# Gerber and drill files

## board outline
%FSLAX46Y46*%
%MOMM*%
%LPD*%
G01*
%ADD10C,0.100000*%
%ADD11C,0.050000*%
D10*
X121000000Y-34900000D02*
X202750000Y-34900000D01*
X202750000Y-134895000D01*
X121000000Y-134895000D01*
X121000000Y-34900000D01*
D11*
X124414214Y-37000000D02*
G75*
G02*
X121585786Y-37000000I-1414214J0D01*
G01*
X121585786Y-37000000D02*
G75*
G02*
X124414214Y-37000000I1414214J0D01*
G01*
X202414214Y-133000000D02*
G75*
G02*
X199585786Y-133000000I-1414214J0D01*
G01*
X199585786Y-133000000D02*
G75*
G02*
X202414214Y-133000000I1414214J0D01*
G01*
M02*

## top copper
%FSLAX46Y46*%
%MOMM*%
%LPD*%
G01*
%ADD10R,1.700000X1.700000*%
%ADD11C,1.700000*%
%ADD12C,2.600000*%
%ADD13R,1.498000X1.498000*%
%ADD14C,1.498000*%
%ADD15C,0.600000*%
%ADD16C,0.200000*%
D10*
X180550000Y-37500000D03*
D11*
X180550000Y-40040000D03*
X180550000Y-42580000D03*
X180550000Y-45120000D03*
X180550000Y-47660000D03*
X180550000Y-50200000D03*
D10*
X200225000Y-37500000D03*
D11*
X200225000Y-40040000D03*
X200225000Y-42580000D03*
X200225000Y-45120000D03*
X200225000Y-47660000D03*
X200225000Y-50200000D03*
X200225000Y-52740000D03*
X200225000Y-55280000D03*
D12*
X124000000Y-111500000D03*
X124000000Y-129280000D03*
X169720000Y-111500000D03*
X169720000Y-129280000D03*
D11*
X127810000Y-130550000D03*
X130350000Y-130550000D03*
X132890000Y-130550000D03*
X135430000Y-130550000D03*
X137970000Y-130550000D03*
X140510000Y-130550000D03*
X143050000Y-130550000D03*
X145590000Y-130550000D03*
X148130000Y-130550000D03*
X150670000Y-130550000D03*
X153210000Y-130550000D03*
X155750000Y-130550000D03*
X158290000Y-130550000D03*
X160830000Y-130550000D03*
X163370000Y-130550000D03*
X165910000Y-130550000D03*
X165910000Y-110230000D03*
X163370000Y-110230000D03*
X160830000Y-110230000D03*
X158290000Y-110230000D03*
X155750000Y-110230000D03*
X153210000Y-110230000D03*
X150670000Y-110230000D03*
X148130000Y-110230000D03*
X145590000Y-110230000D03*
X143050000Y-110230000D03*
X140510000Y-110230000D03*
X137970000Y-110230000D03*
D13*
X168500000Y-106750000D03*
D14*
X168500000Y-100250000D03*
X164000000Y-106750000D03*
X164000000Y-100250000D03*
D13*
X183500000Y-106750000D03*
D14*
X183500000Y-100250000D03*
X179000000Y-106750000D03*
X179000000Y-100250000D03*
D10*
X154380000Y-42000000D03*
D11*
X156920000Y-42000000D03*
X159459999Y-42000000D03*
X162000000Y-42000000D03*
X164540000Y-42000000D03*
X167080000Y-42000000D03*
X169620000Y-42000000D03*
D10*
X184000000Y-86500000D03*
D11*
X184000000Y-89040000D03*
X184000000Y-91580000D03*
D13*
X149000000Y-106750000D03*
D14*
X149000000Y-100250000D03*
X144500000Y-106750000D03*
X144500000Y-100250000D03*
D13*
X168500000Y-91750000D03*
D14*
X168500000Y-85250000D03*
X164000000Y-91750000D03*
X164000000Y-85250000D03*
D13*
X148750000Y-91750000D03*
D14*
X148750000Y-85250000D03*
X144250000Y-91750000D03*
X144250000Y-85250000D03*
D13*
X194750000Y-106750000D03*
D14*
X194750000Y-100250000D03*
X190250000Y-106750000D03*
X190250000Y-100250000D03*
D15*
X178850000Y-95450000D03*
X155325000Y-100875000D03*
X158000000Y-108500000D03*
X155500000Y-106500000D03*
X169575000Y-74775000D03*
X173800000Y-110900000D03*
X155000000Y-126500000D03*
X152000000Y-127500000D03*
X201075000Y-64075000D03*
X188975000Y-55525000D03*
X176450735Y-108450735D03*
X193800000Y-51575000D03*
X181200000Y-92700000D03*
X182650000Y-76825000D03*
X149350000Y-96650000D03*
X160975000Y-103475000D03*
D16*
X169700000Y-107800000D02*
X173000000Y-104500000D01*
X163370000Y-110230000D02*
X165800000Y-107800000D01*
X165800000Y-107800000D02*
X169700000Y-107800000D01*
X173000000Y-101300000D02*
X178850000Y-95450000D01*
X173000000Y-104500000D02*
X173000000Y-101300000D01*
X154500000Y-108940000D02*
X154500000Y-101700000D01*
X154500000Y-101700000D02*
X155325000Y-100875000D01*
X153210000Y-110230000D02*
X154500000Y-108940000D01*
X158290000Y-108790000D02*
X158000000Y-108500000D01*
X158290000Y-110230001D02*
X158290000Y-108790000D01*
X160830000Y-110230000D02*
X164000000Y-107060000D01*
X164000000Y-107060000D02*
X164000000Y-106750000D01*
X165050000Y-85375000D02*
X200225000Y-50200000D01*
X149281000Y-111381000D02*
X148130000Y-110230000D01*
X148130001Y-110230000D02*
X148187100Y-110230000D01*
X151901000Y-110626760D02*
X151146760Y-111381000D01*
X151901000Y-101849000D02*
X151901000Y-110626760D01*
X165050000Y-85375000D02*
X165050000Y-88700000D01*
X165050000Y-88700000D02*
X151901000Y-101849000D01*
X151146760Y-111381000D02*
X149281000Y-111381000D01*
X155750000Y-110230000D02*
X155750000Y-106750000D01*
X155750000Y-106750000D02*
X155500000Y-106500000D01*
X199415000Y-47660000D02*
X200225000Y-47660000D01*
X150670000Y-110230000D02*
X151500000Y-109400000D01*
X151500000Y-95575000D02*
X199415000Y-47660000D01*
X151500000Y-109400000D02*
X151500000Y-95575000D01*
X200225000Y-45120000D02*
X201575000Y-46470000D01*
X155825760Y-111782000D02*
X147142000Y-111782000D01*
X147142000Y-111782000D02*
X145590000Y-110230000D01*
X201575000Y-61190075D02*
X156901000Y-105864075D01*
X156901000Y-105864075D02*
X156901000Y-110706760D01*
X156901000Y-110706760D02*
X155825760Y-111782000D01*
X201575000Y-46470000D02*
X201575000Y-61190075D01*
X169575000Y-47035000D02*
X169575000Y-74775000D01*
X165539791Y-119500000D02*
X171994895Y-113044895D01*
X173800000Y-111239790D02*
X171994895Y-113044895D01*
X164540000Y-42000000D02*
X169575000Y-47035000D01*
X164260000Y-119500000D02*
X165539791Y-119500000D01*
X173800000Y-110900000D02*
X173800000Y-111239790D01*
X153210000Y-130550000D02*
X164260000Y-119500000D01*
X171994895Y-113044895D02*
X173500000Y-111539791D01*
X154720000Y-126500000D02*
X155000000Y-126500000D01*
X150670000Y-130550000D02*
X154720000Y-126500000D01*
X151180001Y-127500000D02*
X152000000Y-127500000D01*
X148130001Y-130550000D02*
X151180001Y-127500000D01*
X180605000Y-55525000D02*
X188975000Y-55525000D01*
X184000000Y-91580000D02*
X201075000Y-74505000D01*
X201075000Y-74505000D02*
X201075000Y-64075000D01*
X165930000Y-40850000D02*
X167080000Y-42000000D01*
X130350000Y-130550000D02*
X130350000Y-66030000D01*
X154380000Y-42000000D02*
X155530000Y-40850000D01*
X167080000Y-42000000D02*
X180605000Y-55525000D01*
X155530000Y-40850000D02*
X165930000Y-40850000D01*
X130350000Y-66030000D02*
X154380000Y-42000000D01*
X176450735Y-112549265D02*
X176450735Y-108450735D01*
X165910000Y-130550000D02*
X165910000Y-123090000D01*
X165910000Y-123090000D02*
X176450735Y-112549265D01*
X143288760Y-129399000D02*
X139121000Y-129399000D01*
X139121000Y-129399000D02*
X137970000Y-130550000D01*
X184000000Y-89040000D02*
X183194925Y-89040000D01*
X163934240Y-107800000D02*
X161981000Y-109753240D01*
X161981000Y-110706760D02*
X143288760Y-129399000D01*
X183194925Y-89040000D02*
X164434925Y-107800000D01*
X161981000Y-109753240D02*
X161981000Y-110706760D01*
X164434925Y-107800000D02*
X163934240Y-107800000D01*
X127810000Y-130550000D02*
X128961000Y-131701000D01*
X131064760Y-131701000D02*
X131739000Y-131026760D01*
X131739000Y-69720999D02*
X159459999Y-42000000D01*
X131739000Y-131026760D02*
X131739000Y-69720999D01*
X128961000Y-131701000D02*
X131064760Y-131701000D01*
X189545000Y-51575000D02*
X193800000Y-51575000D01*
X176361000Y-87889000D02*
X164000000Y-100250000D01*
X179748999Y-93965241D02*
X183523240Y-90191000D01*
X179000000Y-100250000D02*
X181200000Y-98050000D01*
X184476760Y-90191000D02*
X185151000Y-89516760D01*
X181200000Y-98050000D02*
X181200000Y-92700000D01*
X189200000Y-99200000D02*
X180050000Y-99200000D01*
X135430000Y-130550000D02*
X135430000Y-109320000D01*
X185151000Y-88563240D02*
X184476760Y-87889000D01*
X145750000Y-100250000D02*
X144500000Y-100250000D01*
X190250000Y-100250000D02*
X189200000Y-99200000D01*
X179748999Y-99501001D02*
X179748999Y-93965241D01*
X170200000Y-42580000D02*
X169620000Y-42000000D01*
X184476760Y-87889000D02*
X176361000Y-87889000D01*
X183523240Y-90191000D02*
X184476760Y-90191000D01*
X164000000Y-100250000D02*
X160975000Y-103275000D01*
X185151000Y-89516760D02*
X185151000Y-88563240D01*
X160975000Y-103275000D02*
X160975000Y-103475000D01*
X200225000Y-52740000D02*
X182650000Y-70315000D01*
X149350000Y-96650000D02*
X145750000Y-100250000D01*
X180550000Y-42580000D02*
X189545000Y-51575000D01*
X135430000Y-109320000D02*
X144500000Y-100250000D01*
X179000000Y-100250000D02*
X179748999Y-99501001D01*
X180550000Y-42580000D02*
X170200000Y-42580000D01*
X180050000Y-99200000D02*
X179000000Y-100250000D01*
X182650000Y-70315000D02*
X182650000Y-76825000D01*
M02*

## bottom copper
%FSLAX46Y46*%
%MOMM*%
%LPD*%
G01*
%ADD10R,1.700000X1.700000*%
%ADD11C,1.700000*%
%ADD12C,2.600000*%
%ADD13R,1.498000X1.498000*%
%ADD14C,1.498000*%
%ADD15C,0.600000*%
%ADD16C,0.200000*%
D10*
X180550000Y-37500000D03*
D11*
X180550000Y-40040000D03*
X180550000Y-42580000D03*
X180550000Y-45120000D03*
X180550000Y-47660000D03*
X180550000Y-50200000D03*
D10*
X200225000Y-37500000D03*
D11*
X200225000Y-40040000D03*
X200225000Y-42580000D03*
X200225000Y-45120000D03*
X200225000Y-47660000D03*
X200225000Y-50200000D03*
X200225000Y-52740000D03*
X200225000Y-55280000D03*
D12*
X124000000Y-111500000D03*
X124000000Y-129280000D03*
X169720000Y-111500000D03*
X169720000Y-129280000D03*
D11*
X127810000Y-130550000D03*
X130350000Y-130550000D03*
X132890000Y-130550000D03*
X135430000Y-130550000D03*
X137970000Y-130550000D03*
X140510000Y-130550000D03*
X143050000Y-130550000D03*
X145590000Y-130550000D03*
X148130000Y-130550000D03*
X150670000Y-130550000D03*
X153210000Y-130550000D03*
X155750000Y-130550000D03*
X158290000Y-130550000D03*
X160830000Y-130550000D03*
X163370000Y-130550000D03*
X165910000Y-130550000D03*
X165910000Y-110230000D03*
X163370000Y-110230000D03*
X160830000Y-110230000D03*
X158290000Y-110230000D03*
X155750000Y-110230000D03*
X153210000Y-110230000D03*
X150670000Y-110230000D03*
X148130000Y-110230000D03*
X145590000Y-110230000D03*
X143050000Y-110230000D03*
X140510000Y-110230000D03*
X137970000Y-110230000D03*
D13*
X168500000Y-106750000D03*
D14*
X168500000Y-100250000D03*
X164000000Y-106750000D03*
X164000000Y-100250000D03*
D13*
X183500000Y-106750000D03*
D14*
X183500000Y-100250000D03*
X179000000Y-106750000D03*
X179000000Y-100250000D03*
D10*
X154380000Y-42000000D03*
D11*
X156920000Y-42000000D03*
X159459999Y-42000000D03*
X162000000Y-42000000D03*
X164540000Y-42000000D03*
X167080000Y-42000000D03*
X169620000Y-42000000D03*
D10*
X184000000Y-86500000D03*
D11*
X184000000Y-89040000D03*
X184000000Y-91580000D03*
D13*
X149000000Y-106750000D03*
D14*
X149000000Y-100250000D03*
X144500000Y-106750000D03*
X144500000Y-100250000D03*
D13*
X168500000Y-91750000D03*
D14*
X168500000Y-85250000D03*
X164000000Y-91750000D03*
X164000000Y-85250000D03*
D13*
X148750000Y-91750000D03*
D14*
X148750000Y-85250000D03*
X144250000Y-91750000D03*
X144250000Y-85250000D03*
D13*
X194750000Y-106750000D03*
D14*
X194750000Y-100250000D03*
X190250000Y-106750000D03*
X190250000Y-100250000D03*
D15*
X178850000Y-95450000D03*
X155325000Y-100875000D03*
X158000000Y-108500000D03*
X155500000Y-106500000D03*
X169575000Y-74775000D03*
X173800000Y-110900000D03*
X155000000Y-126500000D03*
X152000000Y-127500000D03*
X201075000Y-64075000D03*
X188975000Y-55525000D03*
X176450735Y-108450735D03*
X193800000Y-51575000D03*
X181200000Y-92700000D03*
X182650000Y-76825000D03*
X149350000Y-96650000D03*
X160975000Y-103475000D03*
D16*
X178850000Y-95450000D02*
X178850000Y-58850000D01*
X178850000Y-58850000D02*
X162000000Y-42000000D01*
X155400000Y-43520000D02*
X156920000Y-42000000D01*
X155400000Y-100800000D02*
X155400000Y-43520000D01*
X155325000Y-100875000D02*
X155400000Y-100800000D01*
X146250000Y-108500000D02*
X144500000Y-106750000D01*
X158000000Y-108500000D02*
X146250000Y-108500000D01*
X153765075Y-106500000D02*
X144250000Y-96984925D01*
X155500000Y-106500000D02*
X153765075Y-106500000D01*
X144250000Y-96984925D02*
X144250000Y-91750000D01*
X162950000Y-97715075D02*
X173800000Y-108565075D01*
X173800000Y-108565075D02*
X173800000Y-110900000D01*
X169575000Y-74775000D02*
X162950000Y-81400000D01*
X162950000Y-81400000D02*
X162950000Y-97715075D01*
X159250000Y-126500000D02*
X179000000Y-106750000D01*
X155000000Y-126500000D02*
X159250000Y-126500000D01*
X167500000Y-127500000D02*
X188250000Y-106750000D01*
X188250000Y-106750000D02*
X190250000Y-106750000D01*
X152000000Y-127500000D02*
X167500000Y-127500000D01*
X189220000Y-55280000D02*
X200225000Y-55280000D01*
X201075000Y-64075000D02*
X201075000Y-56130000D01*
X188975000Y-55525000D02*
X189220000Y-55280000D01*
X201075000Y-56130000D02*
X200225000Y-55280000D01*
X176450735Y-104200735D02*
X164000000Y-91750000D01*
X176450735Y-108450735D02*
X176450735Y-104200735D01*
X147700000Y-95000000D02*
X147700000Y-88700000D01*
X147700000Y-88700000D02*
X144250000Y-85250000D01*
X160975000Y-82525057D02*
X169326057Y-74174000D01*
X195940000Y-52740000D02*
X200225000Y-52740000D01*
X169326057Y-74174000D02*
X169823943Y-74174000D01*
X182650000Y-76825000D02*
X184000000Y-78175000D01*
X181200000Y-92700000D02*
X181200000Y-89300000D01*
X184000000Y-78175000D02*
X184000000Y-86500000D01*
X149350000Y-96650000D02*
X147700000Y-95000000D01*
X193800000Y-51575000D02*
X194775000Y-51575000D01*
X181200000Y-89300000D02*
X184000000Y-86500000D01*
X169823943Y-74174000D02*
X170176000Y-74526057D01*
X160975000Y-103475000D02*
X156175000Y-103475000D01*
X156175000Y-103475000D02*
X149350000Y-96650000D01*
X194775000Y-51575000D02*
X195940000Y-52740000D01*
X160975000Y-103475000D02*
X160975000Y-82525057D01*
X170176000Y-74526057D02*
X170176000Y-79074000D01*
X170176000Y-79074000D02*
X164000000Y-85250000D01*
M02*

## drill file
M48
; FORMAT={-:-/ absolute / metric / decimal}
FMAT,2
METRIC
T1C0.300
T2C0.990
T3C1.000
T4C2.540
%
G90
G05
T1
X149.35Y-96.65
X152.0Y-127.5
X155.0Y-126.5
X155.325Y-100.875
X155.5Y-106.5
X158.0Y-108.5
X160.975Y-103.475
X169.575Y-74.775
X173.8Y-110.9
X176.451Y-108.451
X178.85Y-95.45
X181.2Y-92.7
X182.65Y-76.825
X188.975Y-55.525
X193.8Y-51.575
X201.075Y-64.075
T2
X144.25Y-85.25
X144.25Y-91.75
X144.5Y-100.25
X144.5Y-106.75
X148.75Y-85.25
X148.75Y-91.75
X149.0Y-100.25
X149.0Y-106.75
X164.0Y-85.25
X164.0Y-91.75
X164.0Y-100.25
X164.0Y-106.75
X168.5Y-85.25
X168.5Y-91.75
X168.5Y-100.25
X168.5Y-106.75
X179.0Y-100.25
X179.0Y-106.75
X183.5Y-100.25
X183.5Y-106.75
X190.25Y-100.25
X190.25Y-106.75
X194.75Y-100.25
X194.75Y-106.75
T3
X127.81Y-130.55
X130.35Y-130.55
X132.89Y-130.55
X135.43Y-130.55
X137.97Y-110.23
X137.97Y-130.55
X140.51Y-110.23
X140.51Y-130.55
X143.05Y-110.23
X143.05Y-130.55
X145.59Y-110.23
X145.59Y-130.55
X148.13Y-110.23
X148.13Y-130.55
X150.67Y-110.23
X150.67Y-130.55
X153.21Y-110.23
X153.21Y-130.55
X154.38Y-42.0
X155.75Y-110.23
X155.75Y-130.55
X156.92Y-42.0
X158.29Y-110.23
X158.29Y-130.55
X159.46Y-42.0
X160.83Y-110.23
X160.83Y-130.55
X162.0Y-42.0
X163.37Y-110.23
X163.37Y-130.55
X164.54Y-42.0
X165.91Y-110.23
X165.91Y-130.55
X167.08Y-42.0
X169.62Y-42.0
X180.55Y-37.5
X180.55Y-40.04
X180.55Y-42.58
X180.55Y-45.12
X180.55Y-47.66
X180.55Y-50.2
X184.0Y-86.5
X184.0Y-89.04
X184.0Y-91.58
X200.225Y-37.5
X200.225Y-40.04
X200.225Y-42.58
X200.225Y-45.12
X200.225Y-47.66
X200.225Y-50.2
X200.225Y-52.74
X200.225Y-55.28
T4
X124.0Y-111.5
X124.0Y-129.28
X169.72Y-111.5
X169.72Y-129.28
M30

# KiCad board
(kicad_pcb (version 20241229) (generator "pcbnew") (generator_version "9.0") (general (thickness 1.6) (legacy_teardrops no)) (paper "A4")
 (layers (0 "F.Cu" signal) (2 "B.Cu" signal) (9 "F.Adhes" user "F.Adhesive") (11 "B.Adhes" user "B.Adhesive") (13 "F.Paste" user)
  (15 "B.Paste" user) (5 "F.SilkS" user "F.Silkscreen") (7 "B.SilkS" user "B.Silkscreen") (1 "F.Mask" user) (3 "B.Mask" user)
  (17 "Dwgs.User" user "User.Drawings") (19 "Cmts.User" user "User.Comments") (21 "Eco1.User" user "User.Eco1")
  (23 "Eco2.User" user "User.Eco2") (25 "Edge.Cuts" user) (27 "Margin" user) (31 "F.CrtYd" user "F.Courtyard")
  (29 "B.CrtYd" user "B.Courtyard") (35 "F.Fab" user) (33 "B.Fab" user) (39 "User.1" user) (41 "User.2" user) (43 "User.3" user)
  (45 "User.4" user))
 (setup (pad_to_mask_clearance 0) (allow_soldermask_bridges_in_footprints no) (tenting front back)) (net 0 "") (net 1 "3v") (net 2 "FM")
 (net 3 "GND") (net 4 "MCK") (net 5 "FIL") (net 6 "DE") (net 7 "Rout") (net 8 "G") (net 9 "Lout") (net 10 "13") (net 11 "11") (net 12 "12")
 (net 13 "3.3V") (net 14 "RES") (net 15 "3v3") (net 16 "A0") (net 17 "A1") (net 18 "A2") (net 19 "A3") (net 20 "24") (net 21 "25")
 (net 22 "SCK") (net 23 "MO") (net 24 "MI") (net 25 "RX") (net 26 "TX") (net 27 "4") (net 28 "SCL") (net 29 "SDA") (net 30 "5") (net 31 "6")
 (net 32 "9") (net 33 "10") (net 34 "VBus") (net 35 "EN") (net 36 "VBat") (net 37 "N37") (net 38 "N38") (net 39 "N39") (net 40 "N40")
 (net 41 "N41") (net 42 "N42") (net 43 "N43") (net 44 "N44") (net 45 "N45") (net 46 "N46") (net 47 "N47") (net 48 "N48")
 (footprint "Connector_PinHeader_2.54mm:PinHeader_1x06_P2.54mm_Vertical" (layer "F.Cu") (at 180.55 37.5)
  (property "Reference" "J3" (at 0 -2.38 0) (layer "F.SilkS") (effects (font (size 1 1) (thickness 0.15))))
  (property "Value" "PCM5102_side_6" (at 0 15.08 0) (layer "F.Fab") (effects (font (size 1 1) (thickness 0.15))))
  (pad "1" thru_hole rect (at 0 0) (size 1.7 1.7) (drill 1) (layers "*.Cu" "*.Mask") (remove_unused_layers no) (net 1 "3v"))
  (pad "2" thru_hole circle (at 0 2.54) (size 1.7 1.7) (drill 1) (layers "*.Cu" "*.Mask") (remove_unused_layers no) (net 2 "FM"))
  (pad "3" thru_hole circle (at 0 5.08) (size 1.7 1.7) (drill 1) (layers "*.Cu" "*.Mask") (remove_unused_layers no) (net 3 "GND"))
  (pad "4" thru_hole circle (at 0 7.62) (size 1.7 1.7) (drill 1) (layers "*.Cu" "*.Mask") (remove_unused_layers no) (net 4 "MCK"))
  (pad "5" thru_hole circle (at 0 10.16) (size 1.7 1.7) (drill 1) (layers "*.Cu" "*.Mask") (remove_unused_layers no) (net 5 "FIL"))
  (pad "6" thru_hole circle (at 0 12.7) (size 1.7 1.7) (drill 1) (layers "*.Cu" "*.Mask") (remove_unused_layers no) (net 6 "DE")))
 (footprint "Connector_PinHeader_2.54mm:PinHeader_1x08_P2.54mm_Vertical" (layer "F.Cu") (at 200.225 37.5)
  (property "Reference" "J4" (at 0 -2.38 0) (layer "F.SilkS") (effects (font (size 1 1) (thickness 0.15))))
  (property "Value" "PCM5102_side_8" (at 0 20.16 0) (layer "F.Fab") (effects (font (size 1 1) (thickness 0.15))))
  (pad "1" thru_hole rect (at 0 0) (size 1.7 1.7) (drill 1) (layers "*.Cu" "*.Mask") (remove_unused_layers no) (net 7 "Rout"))
  (pad "2" thru_hole circle (at 0 2.54) (size 1.7 1.7) (drill 1) (layers "*.Cu" "*.Mask") (remove_unused_layers no) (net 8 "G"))
  (pad "3" thru_hole circle (at 0 5.08) (size 1.7 1.7) (drill 1) (layers "*.Cu" "*.Mask") (remove_unused_layers no) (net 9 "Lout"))
  (pad "4" thru_hole circle (at 0 7.62) (size 1.7 1.7) (drill 1) (layers "*.Cu" "*.Mask") (remove_unused_layers no) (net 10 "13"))
  (pad "5" thru_hole circle (at 0 10.16) (size 1.7 1.7) (drill 1) (layers "*.Cu" "*.Mask") (remove_unused_layers no) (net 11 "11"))
  (pad "6" thru_hole circle (at 0 12.7) (size 1.7 1.7) (drill 1) (layers "*.Cu" "*.Mask") (remove_unused_layers no) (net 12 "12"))
  (pad "7" thru_hole circle (at 0 15.24) (size 1.7 1.7) (drill 1) (layers "*.Cu" "*.Mask") (remove_unused_layers no) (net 3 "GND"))
  (pad "8" thru_hole circle (at 0 17.78) (size 1.7 1.7) (drill 1) (layers "*.Cu" "*.Mask") (remove_unused_layers no) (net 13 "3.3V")))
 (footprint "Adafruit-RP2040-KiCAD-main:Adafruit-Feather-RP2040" (layer "F.Cu") (at 146.86 120.39)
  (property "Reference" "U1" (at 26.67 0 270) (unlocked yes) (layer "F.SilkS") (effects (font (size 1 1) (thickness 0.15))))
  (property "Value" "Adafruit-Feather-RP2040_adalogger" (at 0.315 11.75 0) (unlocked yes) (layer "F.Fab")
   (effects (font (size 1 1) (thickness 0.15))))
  (pad "" np_thru_hole circle (at -22.86 -8.89) (size 2.6 2.6) (drill 2.54) (layers "*.Cu" "*.Mask") (solder_mask_margin 1.3)
   (clearance 1.3))
  (pad "" np_thru_hole circle (at -22.86 8.89) (size 2.6 2.6) (drill 2.54) (layers "*.Cu" "*.Mask") (solder_mask_margin 1.3) (clearance 1.3))
  (pad "" np_thru_hole circle (at 22.86 -8.89) (size 2.6 2.6) (drill 2.54) (layers "*.Cu" "*.Mask") (solder_mask_margin 1.3) (clearance 1.3))
  (pad "" np_thru_hole circle (at 22.86 8.89) (size 2.6 2.6) (drill 2.54) (layers "*.Cu" "*.Mask") (solder_mask_margin 1.3) (clearance 1.3))
  (pad "1" thru_hole circle (at -19.05 10.16) (size 1.7 1.7) (drill 1) (layers "*.Cu" "*.Mask") (remove_unused_layers no) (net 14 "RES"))
  (pad "2" thru_hole circle (at -16.51 10.16) (size 1.7 1.7) (drill 1) (layers "*.Cu" "*.Mask") (remove_unused_layers no) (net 13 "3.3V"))
  (pad "3" thru_hole circle (at -13.97 10.16) (size 1.7 1.7) (drill 1) (layers "*.Cu" "*.Mask") (remove_unused_layers no) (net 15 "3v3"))
  (pad "4" thru_hole circle (at -11.43 10.16) (size 1.7 1.7) (drill 1) (layers "*.Cu" "*.Mask") (remove_unused_layers no) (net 3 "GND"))
  (pad "5" thru_hole circle (at -8.89 10.16) (size 1.7 1.7) (drill 1) (layers "*.Cu" "*.Mask") (remove_unused_layers no) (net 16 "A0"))
  (pad "6" thru_hole circle (at -6.35 10.16) (size 1.7 1.7) (drill 1) (layers "*.Cu" "*.Mask") (remove_unused_layers no) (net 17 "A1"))
  (pad "7" thru_hole circle (at -3.81 10.16) (size 1.7 1.7) (drill 1) (layers "*.Cu" "*.Mask") (remove_unused_layers no) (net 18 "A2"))
  (pad "8" thru_hole circle (at -1.27 10.16) (size 1.7 1.7) (drill 1) (layers "*.Cu" "*.Mask") (remove_unused_layers no) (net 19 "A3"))
  (pad "9" thru_hole circle (at 1.27 10.16) (size 1.7 1.7) (drill 1) (layers "*.Cu" "*.Mask") (remove_unused_layers no) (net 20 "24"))
  (pad "10" thru_hole circle (at 3.81 10.16) (size 1.7 1.7) (drill 1) (layers "*.Cu" "*.Mask") (remove_unused_layers no) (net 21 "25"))
  (pad "11" thru_hole circle (at 6.35 10.16) (size 1.7 1.7) (drill 1) (layers "*.Cu" "*.Mask") (remove_unused_layers no) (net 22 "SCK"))
  (pad "12" thru_hole circle (at 8.89 10.16) (size 1.7 1.7) (drill 1) (layers "*.Cu" "*.Mask") (remove_unused_layers no) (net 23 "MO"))
  (pad "13" thru_hole circle (at 11.43 10.16) (size 1.7 1.7) (drill 1) (layers "*.Cu" "*.Mask") (remove_unused_layers no) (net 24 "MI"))
  (pad "14" thru_hole circle (at 13.97 10.16) (size 1.7 1.7) (drill 1) (layers "*.Cu" "*.Mask") (remove_unused_layers no) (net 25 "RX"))
  (pad "15" thru_hole circle (at 16.51 10.16) (size 1.7 1.7) (drill 1) (layers "*.Cu" "*.Mask") (remove_unused_layers no) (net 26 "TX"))
  (pad "16" thru_hole circle (at 19.05 10.16) (size 1.7 1.7) (drill 1) (layers "*.Cu" "*.Mask") (remove_unused_layers no) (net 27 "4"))
  (pad "17" thru_hole circle (at 19.05 -10.16) (size 1.7 1.7) (drill 1) (layers "*.Cu" "*.Mask") (remove_unused_layers no) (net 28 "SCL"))
  (pad "18" thru_hole circle (at 16.51 -10.16) (size 1.7 1.7) (drill 1) (layers "*.Cu" "*.Mask") (remove_unused_layers no) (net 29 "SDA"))
  (pad "19" thru_hole circle (at 13.97 -10.16) (size 1.7 1.7) (drill 1) (layers "*.Cu" "*.Mask") (remove_unused_layers no) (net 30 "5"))
  (pad "20" thru_hole circle (at 11.43 -10.16) (size 1.7 1.7) (drill 1) (layers "*.Cu" "*.Mask") (remove_unused_layers no) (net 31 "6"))
  (pad "21" thru_hole circle (at 8.89 -10.16) (size 1.7 1.7) (drill 1) (layers "*.Cu" "*.Mask") (remove_unused_layers no) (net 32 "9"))
  (pad "22" thru_hole circle (at 6.35 -10.16) (size 1.7 1.7) (drill 1) (layers "*.Cu" "*.Mask") (remove_unused_layers no) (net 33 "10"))
  (pad "23" thru_hole circle (at 3.81 -10.16) (size 1.7 1.7) (drill 1) (layers "*.Cu" "*.Mask") (remove_unused_layers no) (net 11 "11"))
  (pad "24" thru_hole circle (at 1.27 -10.16) (size 1.7 1.7) (drill 1) (layers "*.Cu" "*.Mask") (remove_unused_layers no) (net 12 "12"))
  (pad "25" thru_hole circle (at -1.27 -10.16) (size 1.7 1.7) (drill 1) (layers "*.Cu" "*.Mask") (remove_unused_layers no) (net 10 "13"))
  (pad "26" thru_hole circle (at -3.81 -10.16) (size 1.7 1.7) (drill 1) (layers "*.Cu" "*.Mask") (remove_unused_layers no) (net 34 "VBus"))
  (pad "27" thru_hole circle (at -6.35 -10.16) (size 1.7 1.7) (drill 1) (layers "*.Cu" "*.Mask") (remove_unused_layers no) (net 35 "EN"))
  (pad "28" thru_hole circle (at -8.89 -10.16) (size 1.7 1.7) (drill 1) (layers "*.Cu" "*.Mask") (remove_unused_layers no) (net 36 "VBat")))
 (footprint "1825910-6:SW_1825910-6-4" (layer "B.Cu") (at 166.25 103.5 90)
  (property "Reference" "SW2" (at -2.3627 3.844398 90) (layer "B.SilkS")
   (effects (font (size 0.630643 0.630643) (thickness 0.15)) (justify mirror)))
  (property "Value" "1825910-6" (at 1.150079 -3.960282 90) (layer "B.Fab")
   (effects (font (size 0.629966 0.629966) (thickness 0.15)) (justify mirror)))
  (pad "1" thru_hole rect (at -3.25 2.25 90) (size 1.498 1.498) (drill 0.99) (layers "*.Cu" "*.Mask") (remove_unused_layers no)
   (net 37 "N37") (solder_mask_margin 0.102))
  (pad "2" thru_hole circle (at 3.25 2.25 90) (size 1.498 1.498) (drill 0.99) (layers "*.Cu" "*.Mask") (remove_unused_layers no)
   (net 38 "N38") (solder_mask_margin 0.102))
  (pad "3" thru_hole circle (at -3.25 -2.25 90) (size 1.498 1.498) (drill 0.99) (layers "*.Cu" "*.Mask") (remove_unused_layers no)
   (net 30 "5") (solder_mask_margin 0.102))
  (pad "4" thru_hole circle (at 3.25 -2.25 90) (size 1.498 1.498) (drill 0.99) (layers "*.Cu" "*.Mask") (remove_unused_layers no)
   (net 3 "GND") (solder_mask_margin 0.102)))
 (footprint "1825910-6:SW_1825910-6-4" (layer "B.Cu") (at 181.25 103.5 90)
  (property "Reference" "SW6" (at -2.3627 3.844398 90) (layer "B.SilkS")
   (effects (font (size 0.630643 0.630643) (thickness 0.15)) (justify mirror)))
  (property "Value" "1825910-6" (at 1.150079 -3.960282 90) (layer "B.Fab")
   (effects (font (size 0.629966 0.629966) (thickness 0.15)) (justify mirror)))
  (pad "1" thru_hole rect (at -3.25 2.25 90) (size 1.498 1.498) (drill 0.99) (layers "*.Cu" "*.Mask") (remove_unused_layers no)
   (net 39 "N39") (solder_mask_margin 0.102))
  (pad "2" thru_hole circle (at 3.25 2.25 90) (size 1.498 1.498) (drill 0.99) (layers "*.Cu" "*.Mask") (remove_unused_layers no)
   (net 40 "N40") (solder_mask_margin 0.102))
  (pad "3" thru_hole circle (at -3.25 -2.25 90) (size 1.498 1.498) (drill 0.99) (layers "*.Cu" "*.Mask") (remove_unused_layers no)
   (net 21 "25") (solder_mask_margin 0.102))
  (pad "4" thru_hole circle (at 3.25 -2.25 90) (size 1.498 1.498) (drill 0.99) (layers "*.Cu" "*.Mask") (remove_unused_layers no)
   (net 3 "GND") (solder_mask_margin 0.102)))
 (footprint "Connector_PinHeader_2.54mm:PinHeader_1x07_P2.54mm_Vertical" (layer "B.Cu") (at 154.38 42 -90)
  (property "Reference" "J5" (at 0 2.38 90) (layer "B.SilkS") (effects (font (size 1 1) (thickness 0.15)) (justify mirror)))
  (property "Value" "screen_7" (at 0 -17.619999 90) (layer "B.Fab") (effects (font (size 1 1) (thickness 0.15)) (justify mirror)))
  (pad "1" thru_hole rect (at 0 0 270) (size 1.7 1.7) (drill 1) (layers "*.Cu" "*.Mask") (remove_unused_layers no) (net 13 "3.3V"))
  (pad "2" thru_hole circle (at 0 -2.54 270) (size 1.7 1.7) (drill 1) (layers "*.Cu" "*.Mask") (remove_unused_layers no) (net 33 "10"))
  (pad "3" thru_hole circle (at 0 -5.079999 270) (size 1.7 1.7) (drill 1) (layers "*.Cu" "*.Mask") (remove_unused_layers no) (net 14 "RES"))
  (pad "4" thru_hole circle (at 0 -7.62 270) (size 1.7 1.7) (drill 1) (layers "*.Cu" "*.Mask") (remove_unused_layers no) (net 29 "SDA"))
  (pad "5" thru_hole circle (at 0 -10.16 270) (size 1.7 1.7) (drill 1) (layers "*.Cu" "*.Mask") (remove_unused_layers no) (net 22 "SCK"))
  (pad "6" thru_hole circle (at 0 -12.7 270) (size 1.7 1.7) (drill 1) (layers "*.Cu" "*.Mask") (remove_unused_layers no) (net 13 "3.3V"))
  (pad "7" thru_hole circle (at 0 -15.24 270) (size 1.7 1.7) (drill 1) (layers "*.Cu" "*.Mask") (remove_unused_layers no) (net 3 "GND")))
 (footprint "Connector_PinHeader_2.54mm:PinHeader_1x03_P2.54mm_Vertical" (layer "B.Cu") (at 184 86.5 180)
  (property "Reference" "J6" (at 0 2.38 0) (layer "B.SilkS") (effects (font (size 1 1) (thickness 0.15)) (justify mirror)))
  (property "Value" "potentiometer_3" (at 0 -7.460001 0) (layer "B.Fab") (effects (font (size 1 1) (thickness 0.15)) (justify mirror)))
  (pad "1" thru_hole rect (at 0 0 180) (size 1.7 1.7) (drill 1) (layers "*.Cu" "*.Mask") (remove_unused_layers no) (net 3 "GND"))
  (pad "2" thru_hole circle (at 0 -2.54 180) (size 1.7 1.7) (drill 1) (layers "*.Cu" "*.Mask") (remove_unused_layers no) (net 16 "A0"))
  (pad "3" thru_hole circle (at 0 -5.08 180) (size 1.7 1.7) (drill 1) (layers "*.Cu" "*.Mask") (remove_unused_layers no) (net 13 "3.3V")))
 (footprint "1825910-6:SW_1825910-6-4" (layer "B.Cu") (at 146.75 103.5 90)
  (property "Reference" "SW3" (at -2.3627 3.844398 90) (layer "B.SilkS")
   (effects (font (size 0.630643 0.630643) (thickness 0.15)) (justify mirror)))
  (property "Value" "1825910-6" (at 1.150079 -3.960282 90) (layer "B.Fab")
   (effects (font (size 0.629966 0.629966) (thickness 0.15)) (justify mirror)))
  (pad "1" thru_hole rect (at -3.25 2.25 90) (size 1.498 1.498) (drill 0.99) (layers "*.Cu" "*.Mask") (remove_unused_layers no)
   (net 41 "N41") (solder_mask_margin 0.102))
  (pad "2" thru_hole circle (at 3.25 2.25 90) (size 1.498 1.498) (drill 0.99) (layers "*.Cu" "*.Mask") (remove_unused_layers no)
   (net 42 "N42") (solder_mask_margin 0.102))
  (pad "3" thru_hole circle (at -3.25 -2.25 90) (size 1.498 1.498) (drill 0.99) (layers "*.Cu" "*.Mask") (remove_unused_layers no)
   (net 31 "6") (solder_mask_margin 0.102))
  (pad "4" thru_hole circle (at 3.25 -2.25 90) (size 1.498 1.498) (drill 0.99) (layers "*.Cu" "*.Mask") (remove_unused_layers no)
   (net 3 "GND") (solder_mask_margin 0.102)))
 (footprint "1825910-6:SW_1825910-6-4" (layer "B.Cu") (at 166.25 88.5 90)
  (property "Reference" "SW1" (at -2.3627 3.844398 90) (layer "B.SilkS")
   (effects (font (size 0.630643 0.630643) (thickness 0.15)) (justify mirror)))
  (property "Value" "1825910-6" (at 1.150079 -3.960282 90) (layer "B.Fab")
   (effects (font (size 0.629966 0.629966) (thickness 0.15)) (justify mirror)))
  (pad "1" thru_hole rect (at -3.25 2.25 90) (size 1.498 1.498) (drill 0.99) (layers "*.Cu" "*.Mask") (remove_unused_layers no)
   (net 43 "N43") (solder_mask_margin 0.102))
  (pad "2" thru_hole circle (at 3.25 2.25 90) (size 1.498 1.498) (drill 0.99) (layers "*.Cu" "*.Mask") (remove_unused_layers no)
   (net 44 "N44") (solder_mask_margin 0.102))
  (pad "3" thru_hole circle (at -3.25 -2.25 90) (size 1.498 1.498) (drill 0.99) (layers "*.Cu" "*.Mask") (remove_unused_layers no)
   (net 27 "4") (solder_mask_margin 0.102))
  (pad "4" thru_hole circle (at 3.25 -2.25 90) (size 1.498 1.498) (drill 0.99) (layers "*.Cu" "*.Mask") (remove_unused_layers no)
   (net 3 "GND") (solder_mask_margin 0.102)))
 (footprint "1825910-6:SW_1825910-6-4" (layer "B.Cu") (at 146.5 88.5 90)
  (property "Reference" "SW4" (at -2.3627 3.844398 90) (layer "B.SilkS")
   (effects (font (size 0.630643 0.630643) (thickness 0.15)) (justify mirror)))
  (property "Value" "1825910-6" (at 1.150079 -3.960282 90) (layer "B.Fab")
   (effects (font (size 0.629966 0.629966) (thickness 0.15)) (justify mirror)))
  (pad "1" thru_hole rect (at -3.25 2.25 90) (size 1.498 1.498) (drill 0.99) (layers "*.Cu" "*.Mask") (remove_unused_layers no)
   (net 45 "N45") (solder_mask_margin 0.102))
  (pad "2" thru_hole circle (at 3.25 2.25 90) (size 1.498 1.498) (drill 0.99) (layers "*.Cu" "*.Mask") (remove_unused_layers no)
   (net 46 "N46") (solder_mask_margin 0.102))
  (pad "3" thru_hole circle (at -3.25 -2.25 90) (size 1.498 1.498) (drill 0.99) (layers "*.Cu" "*.Mask") (remove_unused_layers no)
   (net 32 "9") (solder_mask_margin 0.102))
  (pad "4" thru_hole circle (at 3.25 -2.25 90) (size 1.498 1.498) (drill 0.99) (layers "*.Cu" "*.Mask") (remove_unused_layers no)
   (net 3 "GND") (solder_mask_margin 0.102)))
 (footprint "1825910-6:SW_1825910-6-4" (layer "B.Cu") (at 192.5 103.5 90)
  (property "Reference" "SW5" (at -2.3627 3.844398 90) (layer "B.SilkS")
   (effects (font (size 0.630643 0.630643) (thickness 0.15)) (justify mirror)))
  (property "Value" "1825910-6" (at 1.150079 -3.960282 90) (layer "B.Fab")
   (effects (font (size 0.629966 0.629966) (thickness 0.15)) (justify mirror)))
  (pad "1" thru_hole rect (at -3.25 2.25 90) (size 1.498 1.498) (drill 0.99) (layers "*.Cu" "*.Mask") (remove_unused_layers no)
   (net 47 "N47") (solder_mask_margin 0.102))
  (pad "2" thru_hole circle (at 3.25 2.25 90) (size 1.498 1.498) (drill 0.99) (layers "*.Cu" "*.Mask") (remove_unused_layers no)
   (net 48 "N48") (solder_mask_margin 0.102))
  (pad "3" thru_hole circle (at -3.25 -2.25 90) (size 1.498 1.498) (drill 0.99) (layers "*.Cu" "*.Mask") (remove_unused_layers no)
   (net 20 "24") (solder_mask_margin 0.102))
  (pad "4" thru_hole circle (at 3.25 -2.25 90) (size 1.498 1.498) (drill 0.99) (layers "*.Cu" "*.Mask") (remove_unused_layers no)
   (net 3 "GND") (solder_mask_margin 0.102)))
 (gr_rect (start 121 34.9) (end 202.75 134.895) (stroke (width 0.1) (type solid)) (fill no) (layer "Edge.Cuts"))
 (gr_circle (center 123 37) (end 124 38) (stroke (width 0.05) (type default)) (fill no) (layer "Edge.Cuts"))
 (gr_circle (center 201 133) (end 202 134) (stroke (width 0.05) (type default)) (fill no) (layer "Edge.Cuts"))
 (segment (start 169.7 107.8) (end 173 104.5) (width 0.2) (layer "F.Cu") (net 29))
 (segment (start 163.37 110.23) (end 165.8 107.8) (width 0.2) (layer "F.Cu") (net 29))
 (segment (start 165.8 107.8) (end 169.7 107.8) (width 0.2) (layer "F.Cu") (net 29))
 (segment (start 173 101.3) (end 178.85 95.45) (width 0.2) (layer "F.Cu") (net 29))
 (segment (start 173 104.5) (end 173 101.3) (width 0.2) (layer "F.Cu") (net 29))
 (via (at 178.85 95.45) (size 0.6) (drill 0.3) (layers "F.Cu" "B.Cu") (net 29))
 (segment (start 178.85 95.45) (end 178.85 58.85) (width 0.2) (layer "B.Cu") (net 29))
 (segment (start 178.85 58.85) (end 162 42) (width 0.2) (layer "B.Cu") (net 29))
 (segment (start 154.5 108.94) (end 154.5 101.7) (width 0.2) (layer "F.Cu") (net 33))
 (segment (start 154.5 101.7) (end 155.325 100.875) (width 0.2) (layer "F.Cu") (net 33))
 (segment (start 153.21 110.23) (end 154.5 108.94) (width 0.2) (layer "F.Cu") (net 33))
 (via (at 155.325 100.875) (size 0.6) (drill 0.3) (layers "F.Cu" "B.Cu") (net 33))
 (segment (start 155.4 43.52) (end 156.92 42) (width 0.2) (layer "B.Cu") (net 33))
 (segment (start 155.4 100.8) (end 155.4 43.52) (width 0.2) (layer "B.Cu") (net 33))
 (segment (start 155.325 100.875) (end 155.4 100.8) (width 0.2) (layer "B.Cu") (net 33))
 (segment (start 158.29 108.79) (end 158 108.5) (width 0.2) (layer "F.Cu") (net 31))
 (segment (start 158.29 110.230001) (end 158.29 108.79) (width 0.2) (layer "F.Cu") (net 31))
 (via (at 158 108.5) (size 0.6) (drill 0.3) (layers "F.Cu" "B.Cu") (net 31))
 (segment (start 146.25 108.5) (end 144.5 106.75) (width 0.2) (layer "B.Cu") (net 31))
 (segment (start 158 108.5) (end 146.25 108.5) (width 0.2) (layer "B.Cu") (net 31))
 (segment (start 160.83 110.23) (end 164 107.06) (width 0.2) (layer "F.Cu") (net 30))
 (segment (start 164 107.06) (end 164 106.75) (width 0.2) (layer "F.Cu") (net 30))
 (segment (start 165.05 85.375) (end 200.225 50.2) (width 0.2) (layer "F.Cu") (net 12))
 (segment (start 149.281 111.381) (end 148.13 110.23) (width 0.2) (layer "F.Cu") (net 12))
 (segment (start 148.130001 110.23) (end 148.1871 110.23) (width 0.2) (layer "F.Cu") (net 12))
 (segment (start 151.901 110.62676) (end 151.14676 111.381) (width 0.2) (layer "F.Cu") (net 12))
 (segment (start 151.901 101.849) (end 151.901 110.62676) (width 0.2) (layer "F.Cu") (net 12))
 (segment (start 165.05 85.375) (end 165.05 88.7) (width 0.2) (layer "F.Cu") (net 12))
 (segment (start 165.05 88.7) (end 151.901 101.849) (width 0.2) (layer "F.Cu") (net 12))
 (segment (start 151.14676 111.381) (end 149.281 111.381) (width 0.2) (layer "F.Cu") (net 12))
 (segment (start 155.75 110.23) (end 155.75 106.75) (width 0.2) (layer "F.Cu") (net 32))
 (segment (start 155.75 106.75) (end 155.5 106.5) (width 0.2) (layer "F.Cu") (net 32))
 (via (at 155.5 106.5) (size 0.6) (drill 0.3) (layers "F.Cu" "B.Cu") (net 32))
 (segment (start 153.765075 106.5) (end 144.25 96.984925) (width 0.2) (layer "B.Cu") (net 32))
 (segment (start 155.5 106.5) (end 153.765075 106.5) (width 0.2) (layer "B.Cu") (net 32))
 (segment (start 144.25 96.984925) (end 144.25 91.75) (width 0.2) (layer "B.Cu") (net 32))
 (segment (start 199.415 47.66) (end 200.225 47.66) (width 0.2) (layer "F.Cu") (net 11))
 (segment (start 150.67 110.23) (end 151.5 109.4) (width 0.2) (layer "F.Cu") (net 11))
 (segment (start 151.5 95.575) (end 199.415 47.66) (width 0.2) (layer "F.Cu") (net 11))
 (segment (start 151.5 109.4) (end 151.5 95.575) (width 0.2) (layer "F.Cu") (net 11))
 (segment (start 200.225 45.12) (end 201.575 46.47) (width 0.2) (layer "F.Cu") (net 10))
 (segment (start 155.82576 111.782) (end 147.142 111.782) (width 0.2) (layer "F.Cu") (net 10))
 (segment (start 147.142 111.782) (end 145.59 110.23) (width 0.2) (layer "F.Cu") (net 10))
 (segment (start 201.575 61.190075) (end 156.901 105.864075) (width 0.2) (layer "F.Cu") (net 10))
 (segment (start 156.901 105.864075) (end 156.901 110.70676) (width 0.2) (layer "F.Cu") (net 10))
 (segment (start 156.901 110.70676) (end 155.82576 111.782) (width 0.2) (layer "F.Cu") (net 10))
 (segment (start 201.575 46.47) (end 201.575 61.190075) (width 0.2) (layer "F.Cu") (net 10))
 (segment (start 169.575 47.035) (end 169.575 74.775) (width 0.2) (layer "F.Cu") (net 22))
 (segment (start 165.539791 119.5) (end 171.994895 113.044895) (width 0.2) (layer "F.Cu") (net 22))
 (segment (start 173.8 111.23979) (end 171.994895 113.044895) (width 0.2) (layer "F.Cu") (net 22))
 (segment (start 164.54 42) (end 169.575 47.035) (width 0.2) (layer "F.Cu") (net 22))
 (segment (start 164.26 119.5) (end 165.539791 119.5) (width 0.2) (layer "F.Cu") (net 22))
 (segment (start 173.8 110.9) (end 173.8 111.23979) (width 0.2) (layer "F.Cu") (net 22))
 (segment (start 153.21 130.55) (end 164.26 119.5) (width 0.2) (layer "F.Cu") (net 22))
 (segment (start 171.994895 113.044895) (end 173.5 111.539791) (width 0.2) (layer "F.Cu") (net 22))
 (via (at 169.575 74.775) (size 0.6) (drill 0.3) (layers "F.Cu" "B.Cu") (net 22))
 (via (at 173.8 110.9) (size 0.6) (drill 0.3) (layers "F.Cu" "B.Cu") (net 22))
 (segment (start 162.95 97.715075) (end 173.8 108.565075) (width 0.2) (layer "B.Cu") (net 22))
 (segment (start 173.8 108.565075) (end 173.8 110.9) (width 0.2) (layer "B.Cu") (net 22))
 (segment (start 169.575 74.775) (end 162.95 81.4) (width 0.2) (layer "B.Cu") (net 22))
 (segment (start 162.95 81.4) (end 162.95 97.715075) (width 0.2) (layer "B.Cu") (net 22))
 (segment (start 154.72 126.5) (end 155 126.5) (width 0.2) (layer "F.Cu") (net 21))
 (segment (start 150.67 130.55) (end 154.72 126.5) (width 0.2) (layer "F.Cu") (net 21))
 (via (at 155 126.5) (size 0.6) (drill 0.3) (layers "F.Cu" "B.Cu") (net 21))
 (segment (start 159.25 126.5) (end 179 106.75) (width 0.2) (layer "B.Cu") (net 21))
 (segment (start 155 126.5) (end 159.25 126.5) (width 0.2) (layer "B.Cu") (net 21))
 (segment (start 151.180001 127.5) (end 152 127.5) (width 0.2) (layer "F.Cu") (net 20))
 (segment (start 148.130001 130.55) (end 151.180001 127.5) (width 0.2) (layer "F.Cu") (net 20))
 (via (at 152 127.5) (size 0.6) (drill 0.3) (layers "F.Cu" "B.Cu") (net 20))
 (segment (start 167.5 127.5) (end 188.25 106.75) (width 0.2) (layer "B.Cu") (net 20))
 (segment (start 188.25 106.75) (end 190.25 106.75) (width 0.2) (layer "B.Cu") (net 20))
 (segment (start 152 127.5) (end 167.5 127.5) (width 0.2) (layer "B.Cu") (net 20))
 (segment (start 180.605 55.525) (end 188.975 55.525) (width 0.2) (layer "F.Cu") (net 13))
 (segment (start 184 91.58) (end 201.075 74.505) (width 0.2) (layer "F.Cu") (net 13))
 (segment (start 201.075 74.505) (end 201.075 64.075) (width 0.2) (layer "F.Cu") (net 13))
 (segment (start 165.93 40.85) (end 167.08 42) (width 0.2) (layer "F.Cu") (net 13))
 (segment (start 130.35 130.55) (end 130.35 66.03) (width 0.2) (layer "F.Cu") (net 13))
 (segment (start 154.38 42) (end 155.53 40.85) (width 0.2) (layer "F.Cu") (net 13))
 (segment (start 167.08 42) (end 180.605 55.525) (width 0.2) (layer "F.Cu") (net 13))
 (segment (start 155.53 40.85) (end 165.93 40.85) (width 0.2) (layer "F.Cu") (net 13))
 (segment (start 130.35 66.03) (end 154.38 42) (width 0.2) (layer "F.Cu") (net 13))
 (via (at 201.075 64.075) (size 0.6) (drill 0.3) (layers "F.Cu" "B.Cu") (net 13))
 (via (at 188.975 55.525) (size 0.6) (drill 0.3) (layers "F.Cu" "B.Cu") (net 13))
 (segment (start 189.22 55.28) (end 200.225 55.28) (width 0.2) (layer "B.Cu") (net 13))
 (segment (start 201.075 64.075) (end 201.075 56.13) (width 0.2) (layer "B.Cu") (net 13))
 (segment (start 188.975 55.525) (end 189.22 55.28) (width 0.2) (layer "B.Cu") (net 13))
 (segment (start 201.075 56.13) (end 200.225 55.28) (width 0.2) (layer "B.Cu") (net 13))
 (segment (start 176.450735 112.549265) (end 176.450735 108.450735) (width 0.2) (layer "F.Cu") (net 27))
 (segment (start 165.91 130.55) (end 165.91 123.09) (width 0.2) (layer "F.Cu") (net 27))
 (segment (start 165.91 123.09) (end 176.450735 112.549265) (width 0.2) (layer "F.Cu") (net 27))
 (via (at 176.450735 108.450735) (size 0.6) (drill 0.3) (layers "F.Cu" "B.Cu") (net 27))
 (segment (start 176.450735 104.200735) (end 164 91.75) (width 0.2) (layer "B.Cu") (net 27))
 (segment (start 176.450735 108.450735) (end 176.450735 104.200735) (width 0.2) (layer "B.Cu") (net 27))
 (segment (start 143.28876 129.399) (end 139.121 129.399) (width 0.2) (layer "F.Cu") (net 16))
 (segment (start 139.121 129.399) (end 137.97 130.55) (width 0.2) (layer "F.Cu") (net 16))
 (segment (start 184 89.04) (end 183.194925 89.04) (width 0.2) (layer "F.Cu") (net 16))
 (segment (start 163.93424 107.8) (end 161.981 109.75324) (width 0.2) (layer "F.Cu") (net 16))
 (segment (start 161.981 110.70676) (end 143.28876 129.399) (width 0.2) (layer "F.Cu") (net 16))
 (segment (start 183.194925 89.04) (end 164.434925 107.8) (width 0.2) (layer "F.Cu") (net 16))
 (segment (start 161.981 109.75324) (end 161.981 110.70676) (width 0.2) (layer "F.Cu") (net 16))
 (segment (start 164.434925 107.8) (end 163.93424 107.8) (width 0.2) (layer "F.Cu") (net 16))
 (segment (start 127.81 130.55) (end 128.961 131.701) (width 0.2) (layer "F.Cu") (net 14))
 (segment (start 131.06476 131.701) (end 131.739 131.02676) (width 0.2) (layer "F.Cu") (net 14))
 (segment (start 131.739 69.720999) (end 159.459999 42) (width 0.2) (layer "F.Cu") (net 14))
 (segment (start 131.739 131.02676) (end 131.739 69.720999) (width 0.2) (layer "F.Cu") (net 14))
 (segment (start 128.961 131.701) (end 131.06476 131.701) (width 0.2) (layer "F.Cu") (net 14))
 (segment (start 189.545 51.575) (end 193.8 51.575) (width 0.2) (layer "F.Cu") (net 3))
 (segment (start 176.361 87.889) (end 164 100.25) (width 0.2) (layer "F.Cu") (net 3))
 (segment (start 179.748999 93.965241) (end 183.52324 90.191) (width 0.2) (layer "F.Cu") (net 3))
 (segment (start 179 100.25) (end 181.2 98.05) (width 0.2) (layer "F.Cu") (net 3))
 (segment (start 184.47676 90.191) (end 185.151 89.51676) (width 0.2) (layer "F.Cu") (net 3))
 (segment (start 181.2 98.05) (end 181.2 92.7) (width 0.2) (layer "F.Cu") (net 3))
 (segment (start 189.2 99.2) (end 180.05 99.2) (width 0.2) (layer "F.Cu") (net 3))
 (segment (start 135.43 130.55) (end 135.43 109.32) (width 0.2) (layer "F.Cu") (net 3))
 (segment (start 185.151 88.56324) (end 184.47676 87.889) (width 0.2) (layer "F.Cu") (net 3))
 (segment (start 145.75 100.25) (end 144.5 100.25) (width 0.2) (layer "F.Cu") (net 3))
 (segment (start 190.25 100.25) (end 189.2 99.2) (width 0.2) (layer "F.Cu") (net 3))
 (segment (start 179.748999 99.501001) (end 179.748999 93.965241) (width 0.2) (layer "F.Cu") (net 3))
 (segment (start 170.2 42.58) (end 169.62 42) (width 0.2) (layer "F.Cu") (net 3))
 (segment (start 184.47676 87.889) (end 176.361 87.889) (width 0.2) (layer "F.Cu") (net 3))
 (segment (start 183.52324 90.191) (end 184.47676 90.191) (width 0.2) (layer "F.Cu") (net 3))
 (segment (start 164 100.25) (end 160.975 103.275) (width 0.2) (layer "F.Cu") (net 3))
 (segment (start 185.151 89.51676) (end 185.151 88.56324) (width 0.2) (layer "F.Cu") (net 3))
 (segment (start 160.975 103.275) (end 160.975 103.475) (width 0.2) (layer "F.Cu") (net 3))
 (segment (start 200.225 52.74) (end 182.65 70.315) (width 0.2) (layer "F.Cu") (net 3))
 (segment (start 149.35 96.65) (end 145.75 100.25) (width 0.2) (layer "F.Cu") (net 3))
 (segment (start 180.55 42.58) (end 189.545 51.575) (width 0.2) (layer "F.Cu") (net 3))
 (segment (start 135.43 109.32) (end 144.5 100.25) (width 0.2) (layer "F.Cu") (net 3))
 (segment (start 179 100.25) (end 179.748999 99.501001) (width 0.2) (layer "F.Cu") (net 3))
 (segment (start 180.55 42.58) (end 170.2 42.58) (width 0.2) (layer "F.Cu") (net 3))
 (segment (start 180.05 99.2) (end 179 100.25) (width 0.2) (layer "F.Cu") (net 3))
 (segment (start 182.65 70.315) (end 182.65 76.825) (width 0.2) (layer "F.Cu") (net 3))
 (via (at 193.8 51.575) (size 0.6) (drill 0.3) (layers "F.Cu" "B.Cu") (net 3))
 (via (at 181.2 92.7) (size 0.6) (drill 0.3) (layers "F.Cu" "B.Cu") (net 3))
 (via (at 182.65 76.825) (size 0.6) (drill 0.3) (layers "F.Cu" "B.Cu") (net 3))
 (via (at 149.35 96.65) (size 0.6) (drill 0.3) (layers "F.Cu" "B.Cu") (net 3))
 (via (at 160.975 103.475) (size 0.6) (drill 0.3) (layers "F.Cu" "B.Cu") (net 3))
 (segment (start 147.7 95) (end 147.7 88.7) (width 0.2) (layer "B.Cu") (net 3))
 (segment (start 147.7 88.7) (end 144.25 85.25) (width 0.2) (layer "B.Cu") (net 3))
 (segment (start 160.975 82.525057) (end 169.326057 74.174) (width 0.2) (layer "B.Cu") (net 3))
 (segment (start 195.94 52.74) (end 200.225 52.74) (width 0.2) (layer "B.Cu") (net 3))
 (segment (start 169.326057 74.174) (end 169.823943 74.174) (width 0.2) (layer "B.Cu") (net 3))
 (segment (start 182.65 76.825) (end 184 78.175) (width 0.2) (layer "B.Cu") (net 3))
 (segment (start 181.2 92.7) (end 181.2 89.3) (width 0.2) (layer "B.Cu") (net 3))
 (segment (start 184 78.175) (end 184 86.5) (width 0.2) (layer "B.Cu") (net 3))
 (segment (start 149.35 96.65) (end 147.7 95) (width 0.2) (layer "B.Cu") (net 3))
 (segment (start 193.8 51.575) (end 194.775 51.575) (width 0.2) (layer "B.Cu") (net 3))
 (segment (start 181.2 89.3) (end 184 86.5) (width 0.2) (layer "B.Cu") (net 3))
 (segment (start 169.823943 74.174) (end 170.176 74.526057) (width 0.2) (layer "B.Cu") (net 3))
 (segment (start 160.975 103.475) (end 156.175 103.475) (width 0.2) (layer "B.Cu") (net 3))
 (segment (start 156.175 103.475) (end 149.35 96.65) (width 0.2) (layer "B.Cu") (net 3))
 (segment (start 194.775 51.575) (end 195.94 52.74) (width 0.2) (layer "B.Cu") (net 3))
 (segment (start 160.975 103.475) (end 160.975 82.525057) (width 0.2) (layer "B.Cu") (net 3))
 (segment (start 170.176 74.526057) (end 170.176 79.074) (width 0.2) (layer "B.Cu") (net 3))
 (segment (start 170.176 79.074) (end 164 85.25) (width 0.2) (layer "B.Cu") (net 3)))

